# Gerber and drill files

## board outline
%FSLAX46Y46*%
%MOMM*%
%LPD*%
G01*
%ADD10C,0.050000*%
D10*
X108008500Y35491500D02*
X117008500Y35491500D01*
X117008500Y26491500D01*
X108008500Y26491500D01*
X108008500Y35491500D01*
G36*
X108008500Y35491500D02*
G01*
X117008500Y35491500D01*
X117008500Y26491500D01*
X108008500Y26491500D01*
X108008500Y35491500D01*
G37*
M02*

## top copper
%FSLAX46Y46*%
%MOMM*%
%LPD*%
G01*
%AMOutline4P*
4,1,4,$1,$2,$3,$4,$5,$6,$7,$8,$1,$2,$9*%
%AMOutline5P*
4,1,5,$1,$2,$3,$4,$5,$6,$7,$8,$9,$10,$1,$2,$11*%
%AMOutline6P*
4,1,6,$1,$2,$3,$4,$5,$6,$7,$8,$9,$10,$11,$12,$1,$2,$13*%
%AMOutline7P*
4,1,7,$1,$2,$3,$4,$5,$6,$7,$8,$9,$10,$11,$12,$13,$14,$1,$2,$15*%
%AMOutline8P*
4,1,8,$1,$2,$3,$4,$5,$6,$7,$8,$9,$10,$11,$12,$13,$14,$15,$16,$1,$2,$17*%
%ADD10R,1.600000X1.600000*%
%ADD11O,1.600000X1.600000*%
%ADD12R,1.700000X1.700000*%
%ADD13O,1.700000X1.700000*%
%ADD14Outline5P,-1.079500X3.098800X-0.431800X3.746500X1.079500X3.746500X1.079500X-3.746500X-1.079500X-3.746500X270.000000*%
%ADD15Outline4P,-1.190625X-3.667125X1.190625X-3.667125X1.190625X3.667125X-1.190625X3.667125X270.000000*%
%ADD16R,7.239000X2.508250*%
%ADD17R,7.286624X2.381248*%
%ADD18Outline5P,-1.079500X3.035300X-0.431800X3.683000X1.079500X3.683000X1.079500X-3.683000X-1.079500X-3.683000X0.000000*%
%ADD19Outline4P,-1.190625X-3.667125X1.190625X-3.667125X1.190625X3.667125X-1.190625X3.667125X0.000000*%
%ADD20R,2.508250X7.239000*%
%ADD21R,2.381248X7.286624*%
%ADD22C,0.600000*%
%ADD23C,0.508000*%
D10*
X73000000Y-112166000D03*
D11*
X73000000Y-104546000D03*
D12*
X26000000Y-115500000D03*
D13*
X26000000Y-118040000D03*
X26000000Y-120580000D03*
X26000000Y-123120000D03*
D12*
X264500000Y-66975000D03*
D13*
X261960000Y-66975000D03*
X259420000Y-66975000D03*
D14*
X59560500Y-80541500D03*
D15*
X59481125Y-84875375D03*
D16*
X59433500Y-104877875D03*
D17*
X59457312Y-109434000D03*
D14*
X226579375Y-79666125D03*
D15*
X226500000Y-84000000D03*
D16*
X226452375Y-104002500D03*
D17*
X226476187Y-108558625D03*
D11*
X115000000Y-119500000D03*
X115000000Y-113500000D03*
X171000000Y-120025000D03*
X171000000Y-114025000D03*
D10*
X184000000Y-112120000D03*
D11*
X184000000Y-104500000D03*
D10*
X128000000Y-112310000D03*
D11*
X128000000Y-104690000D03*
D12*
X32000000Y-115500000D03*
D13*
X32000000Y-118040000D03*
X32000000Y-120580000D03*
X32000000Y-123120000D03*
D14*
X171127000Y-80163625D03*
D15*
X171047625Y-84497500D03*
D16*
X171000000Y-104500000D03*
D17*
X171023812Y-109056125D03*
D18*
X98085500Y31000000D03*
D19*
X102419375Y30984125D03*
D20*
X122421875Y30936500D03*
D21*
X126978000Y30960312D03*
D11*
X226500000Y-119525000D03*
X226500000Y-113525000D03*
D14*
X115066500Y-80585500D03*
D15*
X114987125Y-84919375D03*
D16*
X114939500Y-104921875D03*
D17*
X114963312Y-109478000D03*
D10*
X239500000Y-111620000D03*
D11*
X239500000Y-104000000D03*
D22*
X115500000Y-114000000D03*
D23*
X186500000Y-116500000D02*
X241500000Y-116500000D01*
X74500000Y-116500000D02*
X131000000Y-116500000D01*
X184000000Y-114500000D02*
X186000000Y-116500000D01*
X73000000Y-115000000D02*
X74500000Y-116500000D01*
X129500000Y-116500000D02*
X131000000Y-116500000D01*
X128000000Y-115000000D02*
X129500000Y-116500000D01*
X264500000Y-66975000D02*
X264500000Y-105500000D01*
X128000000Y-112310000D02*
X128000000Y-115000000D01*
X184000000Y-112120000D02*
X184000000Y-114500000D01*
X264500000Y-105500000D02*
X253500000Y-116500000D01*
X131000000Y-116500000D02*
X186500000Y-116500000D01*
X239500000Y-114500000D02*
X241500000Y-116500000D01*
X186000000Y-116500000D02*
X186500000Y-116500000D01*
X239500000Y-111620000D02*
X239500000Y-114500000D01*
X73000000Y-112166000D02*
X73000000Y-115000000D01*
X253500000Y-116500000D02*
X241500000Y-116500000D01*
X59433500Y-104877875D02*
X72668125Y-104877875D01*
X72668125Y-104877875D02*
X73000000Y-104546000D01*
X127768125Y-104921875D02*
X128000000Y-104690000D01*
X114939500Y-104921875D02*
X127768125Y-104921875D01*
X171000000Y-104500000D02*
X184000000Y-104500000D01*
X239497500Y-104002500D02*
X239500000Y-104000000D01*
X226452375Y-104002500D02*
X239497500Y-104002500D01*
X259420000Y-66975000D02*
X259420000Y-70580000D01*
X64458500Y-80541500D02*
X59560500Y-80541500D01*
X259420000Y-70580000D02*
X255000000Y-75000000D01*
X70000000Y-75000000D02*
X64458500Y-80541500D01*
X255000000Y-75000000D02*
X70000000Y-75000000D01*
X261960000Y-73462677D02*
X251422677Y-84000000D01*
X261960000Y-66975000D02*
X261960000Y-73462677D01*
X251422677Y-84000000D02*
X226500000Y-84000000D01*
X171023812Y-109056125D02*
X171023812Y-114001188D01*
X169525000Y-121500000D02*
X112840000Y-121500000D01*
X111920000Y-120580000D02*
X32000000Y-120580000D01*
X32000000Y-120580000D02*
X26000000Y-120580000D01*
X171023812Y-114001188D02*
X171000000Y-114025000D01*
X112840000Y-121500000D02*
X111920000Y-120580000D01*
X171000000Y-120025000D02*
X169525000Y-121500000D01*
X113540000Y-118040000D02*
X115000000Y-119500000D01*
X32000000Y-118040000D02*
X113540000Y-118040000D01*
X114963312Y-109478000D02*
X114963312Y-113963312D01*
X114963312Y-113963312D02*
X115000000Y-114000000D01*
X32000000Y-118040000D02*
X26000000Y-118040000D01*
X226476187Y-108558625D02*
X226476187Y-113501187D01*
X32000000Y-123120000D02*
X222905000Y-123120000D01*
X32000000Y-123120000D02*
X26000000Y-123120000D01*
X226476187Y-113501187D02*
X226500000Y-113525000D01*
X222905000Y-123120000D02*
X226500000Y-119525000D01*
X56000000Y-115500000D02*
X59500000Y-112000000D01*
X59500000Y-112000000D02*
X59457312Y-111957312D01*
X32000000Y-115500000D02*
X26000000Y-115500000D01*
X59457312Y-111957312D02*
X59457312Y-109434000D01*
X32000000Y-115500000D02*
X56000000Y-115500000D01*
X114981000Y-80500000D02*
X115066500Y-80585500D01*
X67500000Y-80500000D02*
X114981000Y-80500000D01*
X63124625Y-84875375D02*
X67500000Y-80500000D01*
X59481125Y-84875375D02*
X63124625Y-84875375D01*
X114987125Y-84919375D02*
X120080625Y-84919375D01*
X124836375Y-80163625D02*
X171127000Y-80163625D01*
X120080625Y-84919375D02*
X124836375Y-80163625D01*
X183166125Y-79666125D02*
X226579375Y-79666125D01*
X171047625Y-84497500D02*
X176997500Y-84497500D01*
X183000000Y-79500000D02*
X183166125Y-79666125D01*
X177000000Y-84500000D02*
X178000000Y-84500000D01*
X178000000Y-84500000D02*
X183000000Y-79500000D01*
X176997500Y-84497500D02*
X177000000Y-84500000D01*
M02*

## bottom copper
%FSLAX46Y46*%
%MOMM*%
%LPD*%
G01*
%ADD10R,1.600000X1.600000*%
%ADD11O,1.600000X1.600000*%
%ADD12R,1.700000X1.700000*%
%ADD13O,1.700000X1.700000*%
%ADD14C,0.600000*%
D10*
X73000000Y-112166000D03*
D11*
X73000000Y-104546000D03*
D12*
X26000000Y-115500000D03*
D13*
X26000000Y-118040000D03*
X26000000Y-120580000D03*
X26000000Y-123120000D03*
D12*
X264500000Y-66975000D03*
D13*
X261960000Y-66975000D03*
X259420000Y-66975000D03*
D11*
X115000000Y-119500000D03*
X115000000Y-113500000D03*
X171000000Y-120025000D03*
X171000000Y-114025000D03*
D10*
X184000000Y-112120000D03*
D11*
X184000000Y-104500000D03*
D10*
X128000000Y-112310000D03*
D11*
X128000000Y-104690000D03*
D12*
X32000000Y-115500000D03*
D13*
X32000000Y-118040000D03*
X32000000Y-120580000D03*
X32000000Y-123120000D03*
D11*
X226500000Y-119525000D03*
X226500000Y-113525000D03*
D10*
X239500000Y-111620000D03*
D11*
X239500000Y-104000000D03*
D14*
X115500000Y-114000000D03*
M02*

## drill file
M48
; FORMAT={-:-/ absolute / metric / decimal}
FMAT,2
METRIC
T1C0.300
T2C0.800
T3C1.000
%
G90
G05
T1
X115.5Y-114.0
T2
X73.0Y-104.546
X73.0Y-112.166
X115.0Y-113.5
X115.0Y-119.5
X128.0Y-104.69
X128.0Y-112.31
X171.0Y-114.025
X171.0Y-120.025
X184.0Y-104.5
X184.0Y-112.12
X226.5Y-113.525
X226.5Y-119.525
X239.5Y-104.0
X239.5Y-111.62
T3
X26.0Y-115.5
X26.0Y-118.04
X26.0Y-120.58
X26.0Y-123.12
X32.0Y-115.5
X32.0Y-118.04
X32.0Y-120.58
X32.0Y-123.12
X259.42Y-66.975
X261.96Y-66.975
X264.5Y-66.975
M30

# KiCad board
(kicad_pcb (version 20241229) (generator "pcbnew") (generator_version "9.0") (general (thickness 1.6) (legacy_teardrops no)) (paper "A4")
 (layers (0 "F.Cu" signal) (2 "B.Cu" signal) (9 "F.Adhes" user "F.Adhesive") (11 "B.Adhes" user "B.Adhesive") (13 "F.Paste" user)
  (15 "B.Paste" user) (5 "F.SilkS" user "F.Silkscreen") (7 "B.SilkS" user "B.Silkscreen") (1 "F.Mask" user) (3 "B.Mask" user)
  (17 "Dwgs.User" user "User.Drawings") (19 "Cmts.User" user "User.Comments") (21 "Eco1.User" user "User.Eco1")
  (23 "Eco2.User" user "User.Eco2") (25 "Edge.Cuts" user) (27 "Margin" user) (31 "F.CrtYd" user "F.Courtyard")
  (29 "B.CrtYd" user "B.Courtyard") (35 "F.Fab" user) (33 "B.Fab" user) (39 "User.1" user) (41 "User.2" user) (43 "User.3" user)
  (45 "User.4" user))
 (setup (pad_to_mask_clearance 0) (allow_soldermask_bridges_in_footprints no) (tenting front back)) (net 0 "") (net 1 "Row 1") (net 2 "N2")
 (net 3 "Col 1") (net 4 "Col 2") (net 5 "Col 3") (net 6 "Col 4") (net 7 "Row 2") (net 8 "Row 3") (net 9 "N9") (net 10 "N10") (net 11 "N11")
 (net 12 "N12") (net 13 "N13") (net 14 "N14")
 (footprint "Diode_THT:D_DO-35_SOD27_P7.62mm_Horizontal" (layer "F.Cu") (at 73 112.166 90)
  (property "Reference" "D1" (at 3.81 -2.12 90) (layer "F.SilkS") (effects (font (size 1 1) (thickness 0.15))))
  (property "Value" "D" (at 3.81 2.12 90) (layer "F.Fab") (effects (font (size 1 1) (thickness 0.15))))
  (pad "1" thru_hole rect (at 0 0 90) (size 1.6 1.6) (drill 0.8) (layers "*.Cu" "*.Mask") (remove_unused_layers no) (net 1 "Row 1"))
  (pad "2" thru_hole oval (at 7.62 0 90) (size 1.6 1.6) (drill 0.8) (layers "*.Cu" "*.Mask") (remove_unused_layers no) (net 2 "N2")))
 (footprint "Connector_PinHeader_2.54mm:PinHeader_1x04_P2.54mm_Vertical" (layer "F.Cu") (at 26 115.5)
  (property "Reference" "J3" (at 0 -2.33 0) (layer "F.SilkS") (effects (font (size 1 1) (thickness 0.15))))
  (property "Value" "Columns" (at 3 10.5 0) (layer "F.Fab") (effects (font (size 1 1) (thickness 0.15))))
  (pad "1" thru_hole rect (at 0 0) (size 1.7 1.7) (drill 1) (layers "*.Cu" "*.Mask") (remove_unused_layers no) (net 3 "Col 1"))
  (pad "2" thru_hole oval (at 0 2.54) (size 1.7 1.7) (drill 1) (layers "*.Cu" "*.Mask") (remove_unused_layers no) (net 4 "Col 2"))
  (pad "3" thru_hole oval (at 0 5.08) (size 1.7 1.7) (drill 1) (layers "*.Cu" "*.Mask") (remove_unused_layers no) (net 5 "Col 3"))
  (pad "4" thru_hole oval (at 0 7.62) (size 1.7 1.7) (drill 1) (layers "*.Cu" "*.Mask") (remove_unused_layers no) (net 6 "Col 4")))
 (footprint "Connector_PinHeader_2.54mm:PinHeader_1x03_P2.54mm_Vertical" (layer "F.Cu") (at 264.5 66.975 -90)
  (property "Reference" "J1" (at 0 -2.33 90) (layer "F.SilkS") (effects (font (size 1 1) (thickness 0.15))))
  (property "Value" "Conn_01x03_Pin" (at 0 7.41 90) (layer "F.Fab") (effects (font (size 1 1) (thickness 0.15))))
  (pad "1" thru_hole rect (at 0 0 270) (size 1.7 1.7) (drill 1) (layers "*.Cu" "*.Mask") (remove_unused_layers no) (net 1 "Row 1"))
  (pad "2" thru_hole oval (at 0 2.54 270) (size 1.7 1.7) (drill 1) (layers "*.Cu" "*.Mask") (remove_unused_layers no) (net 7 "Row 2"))
  (pad "3" thru_hole oval (at 0 5.08 270) (size 1.7 1.7) (drill 1) (layers "*.Cu" "*.Mask") (remove_unused_layers no) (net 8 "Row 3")))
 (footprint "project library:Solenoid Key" (layer "F.Cu") (at 59.497 94.956 -90)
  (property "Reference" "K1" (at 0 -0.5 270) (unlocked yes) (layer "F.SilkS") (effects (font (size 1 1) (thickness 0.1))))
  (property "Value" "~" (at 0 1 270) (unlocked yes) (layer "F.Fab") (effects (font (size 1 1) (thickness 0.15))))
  (pad "1" smd roundrect (at -14.4145 -0.0635 270) (size 2.159 7.493) (layers "F.Cu" "F.Mask" "F.Paste") (roundrect_rratio 0)
   (chamfer_ratio 0.3) (chamfer top_left) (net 8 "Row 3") (thermal_bridge_angle 45))
  (pad "2" smd trapezoid (at -10.080625 0.015875 270) (size 2.38125 7.33425) (layers "F.Cu" "F.Mask" "F.Paste") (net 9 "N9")
   (thermal_bridge_angle 45))
  (pad "3" smd rect (at 9.921875 0.0635 270) (size 2.50825 7.239) (layers "F.Cu" "F.Mask" "F.Paste") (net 2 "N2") (thermal_bridge_angle 45))
  (pad "4" smd rect (at 14.478 0.039688 270) (size 2.381248 7.286624) (layers "F.Cu" "F.Mask" "F.Paste") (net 3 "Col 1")
   (thermal_bridge_angle 45)))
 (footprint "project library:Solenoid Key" (layer "F.Cu") (at 226.515875 94.080625 -90)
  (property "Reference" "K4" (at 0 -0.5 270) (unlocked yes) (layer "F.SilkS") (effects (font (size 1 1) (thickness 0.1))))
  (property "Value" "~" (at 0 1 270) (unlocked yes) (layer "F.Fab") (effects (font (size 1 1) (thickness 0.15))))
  (pad "1" smd roundrect (at -14.4145 -0.0635 270) (size 2.159 7.493) (layers "F.Cu" "F.Mask" "F.Paste") (roundrect_rratio 0)
   (chamfer_ratio 0.3) (chamfer top_left) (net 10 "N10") (thermal_bridge_angle 45))
  (pad "2" smd trapezoid (at -10.080625 0.015875 270) (size 2.38125 7.33425) (layers "F.Cu" "F.Mask" "F.Paste") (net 7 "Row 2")
   (thermal_bridge_angle 45))
  (pad "3" smd rect (at 9.921875 0.0635 270) (size 2.50825 7.239) (layers "F.Cu" "F.Mask" "F.Paste") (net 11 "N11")
   (thermal_bridge_angle 45))
  (pad "4" smd rect (at 14.478 0.039688 270) (size 2.381248 7.286624) (layers "F.Cu" "F.Mask" "F.Paste") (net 6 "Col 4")
   (thermal_bridge_angle 45)))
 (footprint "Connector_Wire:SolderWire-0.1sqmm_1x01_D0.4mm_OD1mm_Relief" (layer "F.Cu") (at 115 113.5)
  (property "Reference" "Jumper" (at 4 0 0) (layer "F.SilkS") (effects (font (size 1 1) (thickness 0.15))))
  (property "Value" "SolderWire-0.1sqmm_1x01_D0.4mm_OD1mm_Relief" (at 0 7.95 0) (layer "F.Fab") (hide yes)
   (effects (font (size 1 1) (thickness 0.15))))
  (pad "" thru_hole oval (at 0 6) (size 1.6 1.6) (drill 0.8) (layers "*.Cu" "*.Mask") (remove_unused_layers no) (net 4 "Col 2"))
  (pad "1" thru_hole oval (at 0 0) (size 1.6 1.6) (drill 0.8) (layers "*.Cu" "*.Mask") (remove_unused_layers no) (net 4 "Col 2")))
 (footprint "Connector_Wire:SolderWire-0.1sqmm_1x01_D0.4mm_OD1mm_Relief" (layer "F.Cu") (at 171 114.025)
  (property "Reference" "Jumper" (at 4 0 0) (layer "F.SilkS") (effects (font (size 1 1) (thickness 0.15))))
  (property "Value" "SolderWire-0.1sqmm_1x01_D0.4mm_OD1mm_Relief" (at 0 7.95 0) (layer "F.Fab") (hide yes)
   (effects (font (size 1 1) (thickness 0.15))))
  (pad "" thru_hole oval (at 0 6) (size 1.6 1.6) (drill 0.8) (layers "*.Cu" "*.Mask") (remove_unused_layers no) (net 5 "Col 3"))
  (pad "1" thru_hole oval (at 0 0) (size 1.6 1.6) (drill 0.8) (layers "*.Cu" "*.Mask") (remove_unused_layers no) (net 5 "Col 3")))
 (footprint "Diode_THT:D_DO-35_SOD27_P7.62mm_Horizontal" (layer "F.Cu") (at 184 112.12 90)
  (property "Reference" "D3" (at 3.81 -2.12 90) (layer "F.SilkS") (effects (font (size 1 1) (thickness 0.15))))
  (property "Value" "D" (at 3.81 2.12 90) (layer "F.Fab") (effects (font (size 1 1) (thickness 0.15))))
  (pad "1" thru_hole rect (at 0 0 90) (size 1.6 1.6) (drill 0.8) (layers "*.Cu" "*.Mask") (remove_unused_layers no) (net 1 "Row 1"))
  (pad "2" thru_hole oval (at 7.62 0 90) (size 1.6 1.6) (drill 0.8) (layers "*.Cu" "*.Mask") (remove_unused_layers no) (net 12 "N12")))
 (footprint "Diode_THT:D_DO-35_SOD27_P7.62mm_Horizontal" (layer "F.Cu") (at 128 112.31 90)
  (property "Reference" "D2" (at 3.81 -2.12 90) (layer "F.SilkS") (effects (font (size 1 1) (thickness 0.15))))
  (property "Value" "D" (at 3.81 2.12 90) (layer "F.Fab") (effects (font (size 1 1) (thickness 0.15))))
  (pad "1" thru_hole rect (at 0 0 90) (size 1.6 1.6) (drill 0.8) (layers "*.Cu" "*.Mask") (remove_unused_layers no) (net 1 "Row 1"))
  (pad "2" thru_hole oval (at 7.62 0 90) (size 1.6 1.6) (drill 0.8) (layers "*.Cu" "*.Mask") (remove_unused_layers no) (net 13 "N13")))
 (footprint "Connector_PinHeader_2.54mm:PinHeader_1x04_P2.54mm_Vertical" (layer "F.Cu") (at 32 115.5)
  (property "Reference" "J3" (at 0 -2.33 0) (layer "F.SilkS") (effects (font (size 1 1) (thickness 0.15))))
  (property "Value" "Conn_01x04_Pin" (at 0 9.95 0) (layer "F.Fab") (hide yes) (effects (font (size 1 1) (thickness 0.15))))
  (pad "1" thru_hole rect (at 0 0) (size 1.7 1.7) (drill 1) (layers "*.Cu" "*.Mask") (remove_unused_layers no) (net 3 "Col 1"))
  (pad "2" thru_hole oval (at 0 2.54) (size 1.7 1.7) (drill 1) (layers "*.Cu" "*.Mask") (remove_unused_layers no) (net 4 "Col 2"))
  (pad "3" thru_hole oval (at 0 5.08) (size 1.7 1.7) (drill 1) (layers "*.Cu" "*.Mask") (remove_unused_layers no) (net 5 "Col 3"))
  (pad "4" thru_hole oval (at 0 7.62) (size 1.7 1.7) (drill 1) (layers "*.Cu" "*.Mask") (remove_unused_layers no) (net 6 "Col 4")))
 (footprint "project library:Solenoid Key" (layer "F.Cu") (at 171.0635 94.578125 -90)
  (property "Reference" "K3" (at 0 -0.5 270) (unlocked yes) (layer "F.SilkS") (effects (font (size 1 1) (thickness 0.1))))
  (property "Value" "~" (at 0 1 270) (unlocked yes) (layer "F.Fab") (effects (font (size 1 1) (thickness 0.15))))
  (pad "1" smd roundrect (at -14.4145 -0.0635 270) (size 2.159 7.493) (layers "F.Cu" "F.Mask" "F.Paste") (roundrect_rratio 0)
   (chamfer_ratio 0.3) (chamfer top_left) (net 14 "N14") (thermal_bridge_angle 45))
  (pad "2" smd trapezoid (at -10.080625 0.015875 270) (size 2.38125 7.33425) (layers "F.Cu" "F.Mask" "F.Paste") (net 10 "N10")
   (thermal_bridge_angle 45))
  (pad "3" smd rect (at 9.921875 0.0635 270) (size 2.50825 7.239) (layers "F.Cu" "F.Mask" "F.Paste") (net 12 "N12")
   (thermal_bridge_angle 45))
  (pad "4" smd rect (at 14.478 0.039688 270) (size 2.381248 7.286624) (layers "F.Cu" "F.Mask" "F.Paste") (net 5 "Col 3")
   (thermal_bridge_angle 45)))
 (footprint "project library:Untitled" (layer "F.Cu") (at 112.5 -31)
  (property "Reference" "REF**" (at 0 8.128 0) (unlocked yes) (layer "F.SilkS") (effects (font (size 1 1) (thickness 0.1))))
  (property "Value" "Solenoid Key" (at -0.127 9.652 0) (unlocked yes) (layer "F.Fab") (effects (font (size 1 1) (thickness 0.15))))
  (fp_rect (start -4.4915 -4.4915) (end 4.5085 4.5085) (stroke (width 0.05) (type solid)) (fill yes) (layer "Edge.Cuts"))
  (pad "1" smd roundrect (at -14.4145 0) (size 2.159 7.366) (layers "F.Cu" "F.Mask" "F.Paste") (roundrect_rratio 0) (chamfer_ratio 0.3)
   (chamfer top_left) (thermal_bridge_angle 45))
  (pad "2" smd trapezoid (at -10.080625 0.015875) (size 2.38125 7.33425) (layers "F.Cu" "F.Mask" "F.Paste") (thermal_bridge_angle 45))
  (pad "3" smd rect (at 9.921875 0.0635) (size 2.50825 7.239) (layers "F.Cu" "F.Mask" "F.Paste") (thermal_bridge_angle 45))
  (pad "4" smd rect (at 14.478 0.039688) (size 2.381248 7.286624) (layers "F.Cu" "F.Mask" "F.Paste") (thermal_bridge_angle 45)))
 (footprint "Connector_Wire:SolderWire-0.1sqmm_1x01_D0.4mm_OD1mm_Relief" (layer "F.Cu") (at 226.5 113.525)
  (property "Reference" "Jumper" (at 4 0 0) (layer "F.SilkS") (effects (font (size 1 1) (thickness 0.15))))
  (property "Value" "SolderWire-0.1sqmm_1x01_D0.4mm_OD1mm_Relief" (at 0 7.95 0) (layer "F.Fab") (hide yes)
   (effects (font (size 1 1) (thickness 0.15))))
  (pad "" thru_hole oval (at 0 6) (size 1.6 1.6) (drill 0.8) (layers "*.Cu" "*.Mask") (remove_unused_layers no) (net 6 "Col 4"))
  (pad "1" thru_hole oval (at 0 0) (size 1.6 1.6) (drill 0.8) (layers "*.Cu" "*.Mask") (remove_unused_layers no) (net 6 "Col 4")))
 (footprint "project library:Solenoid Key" (layer "F.Cu") (at 115.003 95 -90)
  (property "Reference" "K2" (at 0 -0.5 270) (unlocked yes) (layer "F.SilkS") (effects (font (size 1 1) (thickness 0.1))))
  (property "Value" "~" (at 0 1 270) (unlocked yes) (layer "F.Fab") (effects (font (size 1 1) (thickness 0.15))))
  (pad "1" smd roundrect (at -14.4145 -0.0635 270) (size 2.159 7.493) (layers "F.Cu" "F.Mask" "F.Paste") (roundrect_rratio 0)
   (chamfer_ratio 0.3) (chamfer top_left) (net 9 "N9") (thermal_bridge_angle 45))
  (pad "2" smd trapezoid (at -10.080625 0.015875 270) (size 2.38125 7.33425) (layers "F.Cu" "F.Mask" "F.Paste") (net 14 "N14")
   (thermal_bridge_angle 45))
  (pad "3" smd rect (at 9.921875 0.0635 270) (size 2.50825 7.239) (layers "F.Cu" "F.Mask" "F.Paste") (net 13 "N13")
   (thermal_bridge_angle 45))
  (pad "4" smd rect (at 14.478 0.039688 270) (size 2.381248 7.286624) (layers "F.Cu" "F.Mask" "F.Paste") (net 4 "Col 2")
   (thermal_bridge_angle 45)))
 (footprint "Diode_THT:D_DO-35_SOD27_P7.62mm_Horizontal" (layer "F.Cu") (at 239.5 111.62 90)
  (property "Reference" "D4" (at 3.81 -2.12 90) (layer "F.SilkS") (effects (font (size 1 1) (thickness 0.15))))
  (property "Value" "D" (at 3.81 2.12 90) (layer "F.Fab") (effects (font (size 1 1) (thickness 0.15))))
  (pad "1" thru_hole rect (at 0 0 90) (size 1.6 1.6) (drill 0.8) (layers "*.Cu" "*.Mask") (remove_unused_layers no) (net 1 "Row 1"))
  (pad "2" thru_hole oval (at 7.62 0 90) (size 1.6 1.6) (drill 0.8) (layers "*.Cu" "*.Mask") (remove_unused_layers no) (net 11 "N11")))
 (segment (start 186.5 116.5) (end 241.5 116.5) (width 0.508) (layer "F.Cu") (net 1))
 (segment (start 74.5 116.5) (end 131 116.5) (width 0.508) (layer "F.Cu") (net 1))
 (segment (start 184 114.5) (end 186 116.5) (width 0.508) (layer "F.Cu") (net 1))
 (segment (start 73 115) (end 74.5 116.5) (width 0.508) (layer "F.Cu") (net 1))
 (segment (start 129.5 116.5) (end 131 116.5) (width 0.508) (layer "F.Cu") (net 1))
 (segment (start 128 115) (end 129.5 116.5) (width 0.508) (layer "F.Cu") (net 1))
 (segment (start 264.5 66.975) (end 264.5 105.5) (width 0.508) (layer "F.Cu") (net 1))
 (segment (start 128 112.31) (end 128 115) (width 0.508) (layer "F.Cu") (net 1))
 (segment (start 184 112.12) (end 184 114.5) (width 0.508) (layer "F.Cu") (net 1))
 (segment (start 264.5 105.5) (end 253.5 116.5) (width 0.508) (layer "F.Cu") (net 1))
 (segment (start 131 116.5) (end 186.5 116.5) (width 0.508) (layer "F.Cu") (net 1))
 (segment (start 239.5 114.5) (end 241.5 116.5) (width 0.508) (layer "F.Cu") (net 1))
 (segment (start 186 116.5) (end 186.5 116.5) (width 0.508) (layer "F.Cu") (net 1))
 (segment (start 239.5 111.62) (end 239.5 114.5) (width 0.508) (layer "F.Cu") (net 1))
 (segment (start 73 112.166) (end 73 115) (width 0.508) (layer "F.Cu") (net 1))
 (segment (start 253.5 116.5) (end 241.5 116.5) (width 0.508) (layer "F.Cu") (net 1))
 (segment (start 59.4335 104.877875) (end 72.668125 104.877875) (width 0.508) (layer "F.Cu") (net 2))
 (segment (start 72.668125 104.877875) (end 73 104.546) (width 0.508) (layer "F.Cu") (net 2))
 (segment (start 127.768125 104.921875) (end 128 104.69) (width 0.508) (layer "F.Cu") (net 13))
 (segment (start 114.9395 104.921875) (end 127.768125 104.921875) (width 0.508) (layer "F.Cu") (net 13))
 (segment (start 171 104.5) (end 184 104.5) (width 0.508) (layer "F.Cu") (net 12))
 (segment (start 239.4975 104.0025) (end 239.5 104) (width 0.508) (layer "F.Cu") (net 11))
 (segment (start 226.452375 104.0025) (end 239.4975 104.0025) (width 0.508) (layer "F.Cu") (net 11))
 (segment (start 259.42 66.975) (end 259.42 70.58) (width 0.508) (layer "F.Cu") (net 8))
 (segment (start 64.4585 80.5415) (end 59.5605 80.5415) (width 0.508) (layer "F.Cu") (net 8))
 (segment (start 259.42 70.58) (end 255 75) (width 0.508) (layer "F.Cu") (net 8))
 (segment (start 70 75) (end 64.4585 80.5415) (width 0.508) (layer "F.Cu") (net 8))
 (segment (start 255 75) (end 70 75) (width 0.508) (layer "F.Cu") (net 8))
 (segment (start 261.96 73.462677) (end 251.422677 84) (width 0.508) (layer "F.Cu") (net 7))
 (segment (start 261.96 66.975) (end 261.96 73.462677) (width 0.508) (layer "F.Cu") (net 7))
 (segment (start 251.422677 84) (end 226.5 84) (width 0.508) (layer "F.Cu") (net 7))
 (segment (start 171.023812 109.056125) (end 171.023812 114.001188) (width 0.508) (layer "F.Cu") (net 5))
 (segment (start 169.525 121.5) (end 112.84 121.5) (width 0.508) (layer "F.Cu") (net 5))
 (segment (start 111.92 120.58) (end 32 120.58) (width 0.508) (layer "F.Cu") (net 5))
 (segment (start 32 120.58) (end 26 120.58) (width 0.508) (layer "F.Cu") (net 5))
 (segment (start 171.023812 114.001188) (end 171 114.025) (width 0.508) (layer "F.Cu") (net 5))
 (segment (start 112.84 121.5) (end 111.92 120.58) (width 0.508) (layer "F.Cu") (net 5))
 (segment (start 171 120.025) (end 169.525 121.5) (width 0.508) (layer "F.Cu") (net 5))
 (segment (start 113.54 118.04) (end 115 119.5) (width 0.508) (layer "F.Cu") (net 4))
 (segment (start 32 118.04) (end 113.54 118.04) (width 0.508) (layer "F.Cu") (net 4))
 (segment (start 114.963312 109.478) (end 114.963312 113.963312) (width 0.508) (layer "F.Cu") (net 4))
 (segment (start 114.963312 113.963312) (end 115 114) (width 0.508) (layer "F.Cu") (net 4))
 (segment (start 32 118.04) (end 26 118.04) (width 0.508) (layer "F.Cu") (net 4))
 (via (at 115.5 114) (size 0.6) (drill 0.3) (layers "F.Cu" "B.Cu") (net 4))
 (segment (start 226.476187 108.558625) (end 226.476187 113.501187) (width 0.508) (layer "F.Cu") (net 6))
 (segment (start 32 123.12) (end 222.905 123.12) (width 0.508) (layer "F.Cu") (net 6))
 (segment (start 32 123.12) (end 26 123.12) (width 0.508) (layer "F.Cu") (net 6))
 (segment (start 226.476187 113.501187) (end 226.5 113.525) (width 0.508) (layer "F.Cu") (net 6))
 (segment (start 222.905 123.12) (end 226.5 119.525) (width 0.508) (layer "F.Cu") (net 6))
 (segment (start 56 115.5) (end 59.5 112) (width 0.508) (layer "F.Cu") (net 3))
 (segment (start 59.5 112) (end 59.457312 111.957312) (width 0.508) (layer "F.Cu") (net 3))
 (segment (start 32 115.5) (end 26 115.5) (width 0.508) (layer "F.Cu") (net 3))
 (segment (start 59.457312 111.957312) (end 59.457312 109.434) (width 0.508) (layer "F.Cu") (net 3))
 (segment (start 32 115.5) (end 56 115.5) (width 0.508) (layer "F.Cu") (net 3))
 (segment (start 114.981 80.5) (end 115.0665 80.5855) (width 0.508) (layer "F.Cu") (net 9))
 (segment (start 67.5 80.5) (end 114.981 80.5) (width 0.508) (layer "F.Cu") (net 9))
 (segment (start 63.124625 84.875375) (end 67.5 80.5) (width 0.508) (layer "F.Cu") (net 9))
 (segment (start 59.481125 84.875375) (end 63.124625 84.875375) (width 0.508) (layer "F.Cu") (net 9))
 (segment (start 114.987125 84.919375) (end 120.080625 84.919375) (width 0.508) (layer "F.Cu") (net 14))
 (segment (start 124.836375 80.163625) (end 171.127 80.163625) (width 0.508) (layer "F.Cu") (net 14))
 (segment (start 120.080625 84.919375) (end 124.836375 80.163625) (width 0.508) (layer "F.Cu") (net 14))
 (segment (start 183.166125 79.666125) (end 226.579375 79.666125) (width 0.508) (layer "F.Cu") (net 10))
 (segment (start 171.047625 84.4975) (end 176.9975 84.4975) (width 0.508) (layer "F.Cu") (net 10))
 (segment (start 183 79.5) (end 183.166125 79.666125) (width 0.508) (layer "F.Cu") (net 10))
 (segment (start 177 84.5) (end 178 84.5) (width 0.508) (layer "F.Cu") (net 10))
 (segment (start 178 84.5) (end 183 79.5) (width 0.508) (layer "F.Cu") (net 10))
 (segment (start 176.9975 84.4975) (end 177 84.5) (width 0.508) (layer "F.Cu") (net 10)))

